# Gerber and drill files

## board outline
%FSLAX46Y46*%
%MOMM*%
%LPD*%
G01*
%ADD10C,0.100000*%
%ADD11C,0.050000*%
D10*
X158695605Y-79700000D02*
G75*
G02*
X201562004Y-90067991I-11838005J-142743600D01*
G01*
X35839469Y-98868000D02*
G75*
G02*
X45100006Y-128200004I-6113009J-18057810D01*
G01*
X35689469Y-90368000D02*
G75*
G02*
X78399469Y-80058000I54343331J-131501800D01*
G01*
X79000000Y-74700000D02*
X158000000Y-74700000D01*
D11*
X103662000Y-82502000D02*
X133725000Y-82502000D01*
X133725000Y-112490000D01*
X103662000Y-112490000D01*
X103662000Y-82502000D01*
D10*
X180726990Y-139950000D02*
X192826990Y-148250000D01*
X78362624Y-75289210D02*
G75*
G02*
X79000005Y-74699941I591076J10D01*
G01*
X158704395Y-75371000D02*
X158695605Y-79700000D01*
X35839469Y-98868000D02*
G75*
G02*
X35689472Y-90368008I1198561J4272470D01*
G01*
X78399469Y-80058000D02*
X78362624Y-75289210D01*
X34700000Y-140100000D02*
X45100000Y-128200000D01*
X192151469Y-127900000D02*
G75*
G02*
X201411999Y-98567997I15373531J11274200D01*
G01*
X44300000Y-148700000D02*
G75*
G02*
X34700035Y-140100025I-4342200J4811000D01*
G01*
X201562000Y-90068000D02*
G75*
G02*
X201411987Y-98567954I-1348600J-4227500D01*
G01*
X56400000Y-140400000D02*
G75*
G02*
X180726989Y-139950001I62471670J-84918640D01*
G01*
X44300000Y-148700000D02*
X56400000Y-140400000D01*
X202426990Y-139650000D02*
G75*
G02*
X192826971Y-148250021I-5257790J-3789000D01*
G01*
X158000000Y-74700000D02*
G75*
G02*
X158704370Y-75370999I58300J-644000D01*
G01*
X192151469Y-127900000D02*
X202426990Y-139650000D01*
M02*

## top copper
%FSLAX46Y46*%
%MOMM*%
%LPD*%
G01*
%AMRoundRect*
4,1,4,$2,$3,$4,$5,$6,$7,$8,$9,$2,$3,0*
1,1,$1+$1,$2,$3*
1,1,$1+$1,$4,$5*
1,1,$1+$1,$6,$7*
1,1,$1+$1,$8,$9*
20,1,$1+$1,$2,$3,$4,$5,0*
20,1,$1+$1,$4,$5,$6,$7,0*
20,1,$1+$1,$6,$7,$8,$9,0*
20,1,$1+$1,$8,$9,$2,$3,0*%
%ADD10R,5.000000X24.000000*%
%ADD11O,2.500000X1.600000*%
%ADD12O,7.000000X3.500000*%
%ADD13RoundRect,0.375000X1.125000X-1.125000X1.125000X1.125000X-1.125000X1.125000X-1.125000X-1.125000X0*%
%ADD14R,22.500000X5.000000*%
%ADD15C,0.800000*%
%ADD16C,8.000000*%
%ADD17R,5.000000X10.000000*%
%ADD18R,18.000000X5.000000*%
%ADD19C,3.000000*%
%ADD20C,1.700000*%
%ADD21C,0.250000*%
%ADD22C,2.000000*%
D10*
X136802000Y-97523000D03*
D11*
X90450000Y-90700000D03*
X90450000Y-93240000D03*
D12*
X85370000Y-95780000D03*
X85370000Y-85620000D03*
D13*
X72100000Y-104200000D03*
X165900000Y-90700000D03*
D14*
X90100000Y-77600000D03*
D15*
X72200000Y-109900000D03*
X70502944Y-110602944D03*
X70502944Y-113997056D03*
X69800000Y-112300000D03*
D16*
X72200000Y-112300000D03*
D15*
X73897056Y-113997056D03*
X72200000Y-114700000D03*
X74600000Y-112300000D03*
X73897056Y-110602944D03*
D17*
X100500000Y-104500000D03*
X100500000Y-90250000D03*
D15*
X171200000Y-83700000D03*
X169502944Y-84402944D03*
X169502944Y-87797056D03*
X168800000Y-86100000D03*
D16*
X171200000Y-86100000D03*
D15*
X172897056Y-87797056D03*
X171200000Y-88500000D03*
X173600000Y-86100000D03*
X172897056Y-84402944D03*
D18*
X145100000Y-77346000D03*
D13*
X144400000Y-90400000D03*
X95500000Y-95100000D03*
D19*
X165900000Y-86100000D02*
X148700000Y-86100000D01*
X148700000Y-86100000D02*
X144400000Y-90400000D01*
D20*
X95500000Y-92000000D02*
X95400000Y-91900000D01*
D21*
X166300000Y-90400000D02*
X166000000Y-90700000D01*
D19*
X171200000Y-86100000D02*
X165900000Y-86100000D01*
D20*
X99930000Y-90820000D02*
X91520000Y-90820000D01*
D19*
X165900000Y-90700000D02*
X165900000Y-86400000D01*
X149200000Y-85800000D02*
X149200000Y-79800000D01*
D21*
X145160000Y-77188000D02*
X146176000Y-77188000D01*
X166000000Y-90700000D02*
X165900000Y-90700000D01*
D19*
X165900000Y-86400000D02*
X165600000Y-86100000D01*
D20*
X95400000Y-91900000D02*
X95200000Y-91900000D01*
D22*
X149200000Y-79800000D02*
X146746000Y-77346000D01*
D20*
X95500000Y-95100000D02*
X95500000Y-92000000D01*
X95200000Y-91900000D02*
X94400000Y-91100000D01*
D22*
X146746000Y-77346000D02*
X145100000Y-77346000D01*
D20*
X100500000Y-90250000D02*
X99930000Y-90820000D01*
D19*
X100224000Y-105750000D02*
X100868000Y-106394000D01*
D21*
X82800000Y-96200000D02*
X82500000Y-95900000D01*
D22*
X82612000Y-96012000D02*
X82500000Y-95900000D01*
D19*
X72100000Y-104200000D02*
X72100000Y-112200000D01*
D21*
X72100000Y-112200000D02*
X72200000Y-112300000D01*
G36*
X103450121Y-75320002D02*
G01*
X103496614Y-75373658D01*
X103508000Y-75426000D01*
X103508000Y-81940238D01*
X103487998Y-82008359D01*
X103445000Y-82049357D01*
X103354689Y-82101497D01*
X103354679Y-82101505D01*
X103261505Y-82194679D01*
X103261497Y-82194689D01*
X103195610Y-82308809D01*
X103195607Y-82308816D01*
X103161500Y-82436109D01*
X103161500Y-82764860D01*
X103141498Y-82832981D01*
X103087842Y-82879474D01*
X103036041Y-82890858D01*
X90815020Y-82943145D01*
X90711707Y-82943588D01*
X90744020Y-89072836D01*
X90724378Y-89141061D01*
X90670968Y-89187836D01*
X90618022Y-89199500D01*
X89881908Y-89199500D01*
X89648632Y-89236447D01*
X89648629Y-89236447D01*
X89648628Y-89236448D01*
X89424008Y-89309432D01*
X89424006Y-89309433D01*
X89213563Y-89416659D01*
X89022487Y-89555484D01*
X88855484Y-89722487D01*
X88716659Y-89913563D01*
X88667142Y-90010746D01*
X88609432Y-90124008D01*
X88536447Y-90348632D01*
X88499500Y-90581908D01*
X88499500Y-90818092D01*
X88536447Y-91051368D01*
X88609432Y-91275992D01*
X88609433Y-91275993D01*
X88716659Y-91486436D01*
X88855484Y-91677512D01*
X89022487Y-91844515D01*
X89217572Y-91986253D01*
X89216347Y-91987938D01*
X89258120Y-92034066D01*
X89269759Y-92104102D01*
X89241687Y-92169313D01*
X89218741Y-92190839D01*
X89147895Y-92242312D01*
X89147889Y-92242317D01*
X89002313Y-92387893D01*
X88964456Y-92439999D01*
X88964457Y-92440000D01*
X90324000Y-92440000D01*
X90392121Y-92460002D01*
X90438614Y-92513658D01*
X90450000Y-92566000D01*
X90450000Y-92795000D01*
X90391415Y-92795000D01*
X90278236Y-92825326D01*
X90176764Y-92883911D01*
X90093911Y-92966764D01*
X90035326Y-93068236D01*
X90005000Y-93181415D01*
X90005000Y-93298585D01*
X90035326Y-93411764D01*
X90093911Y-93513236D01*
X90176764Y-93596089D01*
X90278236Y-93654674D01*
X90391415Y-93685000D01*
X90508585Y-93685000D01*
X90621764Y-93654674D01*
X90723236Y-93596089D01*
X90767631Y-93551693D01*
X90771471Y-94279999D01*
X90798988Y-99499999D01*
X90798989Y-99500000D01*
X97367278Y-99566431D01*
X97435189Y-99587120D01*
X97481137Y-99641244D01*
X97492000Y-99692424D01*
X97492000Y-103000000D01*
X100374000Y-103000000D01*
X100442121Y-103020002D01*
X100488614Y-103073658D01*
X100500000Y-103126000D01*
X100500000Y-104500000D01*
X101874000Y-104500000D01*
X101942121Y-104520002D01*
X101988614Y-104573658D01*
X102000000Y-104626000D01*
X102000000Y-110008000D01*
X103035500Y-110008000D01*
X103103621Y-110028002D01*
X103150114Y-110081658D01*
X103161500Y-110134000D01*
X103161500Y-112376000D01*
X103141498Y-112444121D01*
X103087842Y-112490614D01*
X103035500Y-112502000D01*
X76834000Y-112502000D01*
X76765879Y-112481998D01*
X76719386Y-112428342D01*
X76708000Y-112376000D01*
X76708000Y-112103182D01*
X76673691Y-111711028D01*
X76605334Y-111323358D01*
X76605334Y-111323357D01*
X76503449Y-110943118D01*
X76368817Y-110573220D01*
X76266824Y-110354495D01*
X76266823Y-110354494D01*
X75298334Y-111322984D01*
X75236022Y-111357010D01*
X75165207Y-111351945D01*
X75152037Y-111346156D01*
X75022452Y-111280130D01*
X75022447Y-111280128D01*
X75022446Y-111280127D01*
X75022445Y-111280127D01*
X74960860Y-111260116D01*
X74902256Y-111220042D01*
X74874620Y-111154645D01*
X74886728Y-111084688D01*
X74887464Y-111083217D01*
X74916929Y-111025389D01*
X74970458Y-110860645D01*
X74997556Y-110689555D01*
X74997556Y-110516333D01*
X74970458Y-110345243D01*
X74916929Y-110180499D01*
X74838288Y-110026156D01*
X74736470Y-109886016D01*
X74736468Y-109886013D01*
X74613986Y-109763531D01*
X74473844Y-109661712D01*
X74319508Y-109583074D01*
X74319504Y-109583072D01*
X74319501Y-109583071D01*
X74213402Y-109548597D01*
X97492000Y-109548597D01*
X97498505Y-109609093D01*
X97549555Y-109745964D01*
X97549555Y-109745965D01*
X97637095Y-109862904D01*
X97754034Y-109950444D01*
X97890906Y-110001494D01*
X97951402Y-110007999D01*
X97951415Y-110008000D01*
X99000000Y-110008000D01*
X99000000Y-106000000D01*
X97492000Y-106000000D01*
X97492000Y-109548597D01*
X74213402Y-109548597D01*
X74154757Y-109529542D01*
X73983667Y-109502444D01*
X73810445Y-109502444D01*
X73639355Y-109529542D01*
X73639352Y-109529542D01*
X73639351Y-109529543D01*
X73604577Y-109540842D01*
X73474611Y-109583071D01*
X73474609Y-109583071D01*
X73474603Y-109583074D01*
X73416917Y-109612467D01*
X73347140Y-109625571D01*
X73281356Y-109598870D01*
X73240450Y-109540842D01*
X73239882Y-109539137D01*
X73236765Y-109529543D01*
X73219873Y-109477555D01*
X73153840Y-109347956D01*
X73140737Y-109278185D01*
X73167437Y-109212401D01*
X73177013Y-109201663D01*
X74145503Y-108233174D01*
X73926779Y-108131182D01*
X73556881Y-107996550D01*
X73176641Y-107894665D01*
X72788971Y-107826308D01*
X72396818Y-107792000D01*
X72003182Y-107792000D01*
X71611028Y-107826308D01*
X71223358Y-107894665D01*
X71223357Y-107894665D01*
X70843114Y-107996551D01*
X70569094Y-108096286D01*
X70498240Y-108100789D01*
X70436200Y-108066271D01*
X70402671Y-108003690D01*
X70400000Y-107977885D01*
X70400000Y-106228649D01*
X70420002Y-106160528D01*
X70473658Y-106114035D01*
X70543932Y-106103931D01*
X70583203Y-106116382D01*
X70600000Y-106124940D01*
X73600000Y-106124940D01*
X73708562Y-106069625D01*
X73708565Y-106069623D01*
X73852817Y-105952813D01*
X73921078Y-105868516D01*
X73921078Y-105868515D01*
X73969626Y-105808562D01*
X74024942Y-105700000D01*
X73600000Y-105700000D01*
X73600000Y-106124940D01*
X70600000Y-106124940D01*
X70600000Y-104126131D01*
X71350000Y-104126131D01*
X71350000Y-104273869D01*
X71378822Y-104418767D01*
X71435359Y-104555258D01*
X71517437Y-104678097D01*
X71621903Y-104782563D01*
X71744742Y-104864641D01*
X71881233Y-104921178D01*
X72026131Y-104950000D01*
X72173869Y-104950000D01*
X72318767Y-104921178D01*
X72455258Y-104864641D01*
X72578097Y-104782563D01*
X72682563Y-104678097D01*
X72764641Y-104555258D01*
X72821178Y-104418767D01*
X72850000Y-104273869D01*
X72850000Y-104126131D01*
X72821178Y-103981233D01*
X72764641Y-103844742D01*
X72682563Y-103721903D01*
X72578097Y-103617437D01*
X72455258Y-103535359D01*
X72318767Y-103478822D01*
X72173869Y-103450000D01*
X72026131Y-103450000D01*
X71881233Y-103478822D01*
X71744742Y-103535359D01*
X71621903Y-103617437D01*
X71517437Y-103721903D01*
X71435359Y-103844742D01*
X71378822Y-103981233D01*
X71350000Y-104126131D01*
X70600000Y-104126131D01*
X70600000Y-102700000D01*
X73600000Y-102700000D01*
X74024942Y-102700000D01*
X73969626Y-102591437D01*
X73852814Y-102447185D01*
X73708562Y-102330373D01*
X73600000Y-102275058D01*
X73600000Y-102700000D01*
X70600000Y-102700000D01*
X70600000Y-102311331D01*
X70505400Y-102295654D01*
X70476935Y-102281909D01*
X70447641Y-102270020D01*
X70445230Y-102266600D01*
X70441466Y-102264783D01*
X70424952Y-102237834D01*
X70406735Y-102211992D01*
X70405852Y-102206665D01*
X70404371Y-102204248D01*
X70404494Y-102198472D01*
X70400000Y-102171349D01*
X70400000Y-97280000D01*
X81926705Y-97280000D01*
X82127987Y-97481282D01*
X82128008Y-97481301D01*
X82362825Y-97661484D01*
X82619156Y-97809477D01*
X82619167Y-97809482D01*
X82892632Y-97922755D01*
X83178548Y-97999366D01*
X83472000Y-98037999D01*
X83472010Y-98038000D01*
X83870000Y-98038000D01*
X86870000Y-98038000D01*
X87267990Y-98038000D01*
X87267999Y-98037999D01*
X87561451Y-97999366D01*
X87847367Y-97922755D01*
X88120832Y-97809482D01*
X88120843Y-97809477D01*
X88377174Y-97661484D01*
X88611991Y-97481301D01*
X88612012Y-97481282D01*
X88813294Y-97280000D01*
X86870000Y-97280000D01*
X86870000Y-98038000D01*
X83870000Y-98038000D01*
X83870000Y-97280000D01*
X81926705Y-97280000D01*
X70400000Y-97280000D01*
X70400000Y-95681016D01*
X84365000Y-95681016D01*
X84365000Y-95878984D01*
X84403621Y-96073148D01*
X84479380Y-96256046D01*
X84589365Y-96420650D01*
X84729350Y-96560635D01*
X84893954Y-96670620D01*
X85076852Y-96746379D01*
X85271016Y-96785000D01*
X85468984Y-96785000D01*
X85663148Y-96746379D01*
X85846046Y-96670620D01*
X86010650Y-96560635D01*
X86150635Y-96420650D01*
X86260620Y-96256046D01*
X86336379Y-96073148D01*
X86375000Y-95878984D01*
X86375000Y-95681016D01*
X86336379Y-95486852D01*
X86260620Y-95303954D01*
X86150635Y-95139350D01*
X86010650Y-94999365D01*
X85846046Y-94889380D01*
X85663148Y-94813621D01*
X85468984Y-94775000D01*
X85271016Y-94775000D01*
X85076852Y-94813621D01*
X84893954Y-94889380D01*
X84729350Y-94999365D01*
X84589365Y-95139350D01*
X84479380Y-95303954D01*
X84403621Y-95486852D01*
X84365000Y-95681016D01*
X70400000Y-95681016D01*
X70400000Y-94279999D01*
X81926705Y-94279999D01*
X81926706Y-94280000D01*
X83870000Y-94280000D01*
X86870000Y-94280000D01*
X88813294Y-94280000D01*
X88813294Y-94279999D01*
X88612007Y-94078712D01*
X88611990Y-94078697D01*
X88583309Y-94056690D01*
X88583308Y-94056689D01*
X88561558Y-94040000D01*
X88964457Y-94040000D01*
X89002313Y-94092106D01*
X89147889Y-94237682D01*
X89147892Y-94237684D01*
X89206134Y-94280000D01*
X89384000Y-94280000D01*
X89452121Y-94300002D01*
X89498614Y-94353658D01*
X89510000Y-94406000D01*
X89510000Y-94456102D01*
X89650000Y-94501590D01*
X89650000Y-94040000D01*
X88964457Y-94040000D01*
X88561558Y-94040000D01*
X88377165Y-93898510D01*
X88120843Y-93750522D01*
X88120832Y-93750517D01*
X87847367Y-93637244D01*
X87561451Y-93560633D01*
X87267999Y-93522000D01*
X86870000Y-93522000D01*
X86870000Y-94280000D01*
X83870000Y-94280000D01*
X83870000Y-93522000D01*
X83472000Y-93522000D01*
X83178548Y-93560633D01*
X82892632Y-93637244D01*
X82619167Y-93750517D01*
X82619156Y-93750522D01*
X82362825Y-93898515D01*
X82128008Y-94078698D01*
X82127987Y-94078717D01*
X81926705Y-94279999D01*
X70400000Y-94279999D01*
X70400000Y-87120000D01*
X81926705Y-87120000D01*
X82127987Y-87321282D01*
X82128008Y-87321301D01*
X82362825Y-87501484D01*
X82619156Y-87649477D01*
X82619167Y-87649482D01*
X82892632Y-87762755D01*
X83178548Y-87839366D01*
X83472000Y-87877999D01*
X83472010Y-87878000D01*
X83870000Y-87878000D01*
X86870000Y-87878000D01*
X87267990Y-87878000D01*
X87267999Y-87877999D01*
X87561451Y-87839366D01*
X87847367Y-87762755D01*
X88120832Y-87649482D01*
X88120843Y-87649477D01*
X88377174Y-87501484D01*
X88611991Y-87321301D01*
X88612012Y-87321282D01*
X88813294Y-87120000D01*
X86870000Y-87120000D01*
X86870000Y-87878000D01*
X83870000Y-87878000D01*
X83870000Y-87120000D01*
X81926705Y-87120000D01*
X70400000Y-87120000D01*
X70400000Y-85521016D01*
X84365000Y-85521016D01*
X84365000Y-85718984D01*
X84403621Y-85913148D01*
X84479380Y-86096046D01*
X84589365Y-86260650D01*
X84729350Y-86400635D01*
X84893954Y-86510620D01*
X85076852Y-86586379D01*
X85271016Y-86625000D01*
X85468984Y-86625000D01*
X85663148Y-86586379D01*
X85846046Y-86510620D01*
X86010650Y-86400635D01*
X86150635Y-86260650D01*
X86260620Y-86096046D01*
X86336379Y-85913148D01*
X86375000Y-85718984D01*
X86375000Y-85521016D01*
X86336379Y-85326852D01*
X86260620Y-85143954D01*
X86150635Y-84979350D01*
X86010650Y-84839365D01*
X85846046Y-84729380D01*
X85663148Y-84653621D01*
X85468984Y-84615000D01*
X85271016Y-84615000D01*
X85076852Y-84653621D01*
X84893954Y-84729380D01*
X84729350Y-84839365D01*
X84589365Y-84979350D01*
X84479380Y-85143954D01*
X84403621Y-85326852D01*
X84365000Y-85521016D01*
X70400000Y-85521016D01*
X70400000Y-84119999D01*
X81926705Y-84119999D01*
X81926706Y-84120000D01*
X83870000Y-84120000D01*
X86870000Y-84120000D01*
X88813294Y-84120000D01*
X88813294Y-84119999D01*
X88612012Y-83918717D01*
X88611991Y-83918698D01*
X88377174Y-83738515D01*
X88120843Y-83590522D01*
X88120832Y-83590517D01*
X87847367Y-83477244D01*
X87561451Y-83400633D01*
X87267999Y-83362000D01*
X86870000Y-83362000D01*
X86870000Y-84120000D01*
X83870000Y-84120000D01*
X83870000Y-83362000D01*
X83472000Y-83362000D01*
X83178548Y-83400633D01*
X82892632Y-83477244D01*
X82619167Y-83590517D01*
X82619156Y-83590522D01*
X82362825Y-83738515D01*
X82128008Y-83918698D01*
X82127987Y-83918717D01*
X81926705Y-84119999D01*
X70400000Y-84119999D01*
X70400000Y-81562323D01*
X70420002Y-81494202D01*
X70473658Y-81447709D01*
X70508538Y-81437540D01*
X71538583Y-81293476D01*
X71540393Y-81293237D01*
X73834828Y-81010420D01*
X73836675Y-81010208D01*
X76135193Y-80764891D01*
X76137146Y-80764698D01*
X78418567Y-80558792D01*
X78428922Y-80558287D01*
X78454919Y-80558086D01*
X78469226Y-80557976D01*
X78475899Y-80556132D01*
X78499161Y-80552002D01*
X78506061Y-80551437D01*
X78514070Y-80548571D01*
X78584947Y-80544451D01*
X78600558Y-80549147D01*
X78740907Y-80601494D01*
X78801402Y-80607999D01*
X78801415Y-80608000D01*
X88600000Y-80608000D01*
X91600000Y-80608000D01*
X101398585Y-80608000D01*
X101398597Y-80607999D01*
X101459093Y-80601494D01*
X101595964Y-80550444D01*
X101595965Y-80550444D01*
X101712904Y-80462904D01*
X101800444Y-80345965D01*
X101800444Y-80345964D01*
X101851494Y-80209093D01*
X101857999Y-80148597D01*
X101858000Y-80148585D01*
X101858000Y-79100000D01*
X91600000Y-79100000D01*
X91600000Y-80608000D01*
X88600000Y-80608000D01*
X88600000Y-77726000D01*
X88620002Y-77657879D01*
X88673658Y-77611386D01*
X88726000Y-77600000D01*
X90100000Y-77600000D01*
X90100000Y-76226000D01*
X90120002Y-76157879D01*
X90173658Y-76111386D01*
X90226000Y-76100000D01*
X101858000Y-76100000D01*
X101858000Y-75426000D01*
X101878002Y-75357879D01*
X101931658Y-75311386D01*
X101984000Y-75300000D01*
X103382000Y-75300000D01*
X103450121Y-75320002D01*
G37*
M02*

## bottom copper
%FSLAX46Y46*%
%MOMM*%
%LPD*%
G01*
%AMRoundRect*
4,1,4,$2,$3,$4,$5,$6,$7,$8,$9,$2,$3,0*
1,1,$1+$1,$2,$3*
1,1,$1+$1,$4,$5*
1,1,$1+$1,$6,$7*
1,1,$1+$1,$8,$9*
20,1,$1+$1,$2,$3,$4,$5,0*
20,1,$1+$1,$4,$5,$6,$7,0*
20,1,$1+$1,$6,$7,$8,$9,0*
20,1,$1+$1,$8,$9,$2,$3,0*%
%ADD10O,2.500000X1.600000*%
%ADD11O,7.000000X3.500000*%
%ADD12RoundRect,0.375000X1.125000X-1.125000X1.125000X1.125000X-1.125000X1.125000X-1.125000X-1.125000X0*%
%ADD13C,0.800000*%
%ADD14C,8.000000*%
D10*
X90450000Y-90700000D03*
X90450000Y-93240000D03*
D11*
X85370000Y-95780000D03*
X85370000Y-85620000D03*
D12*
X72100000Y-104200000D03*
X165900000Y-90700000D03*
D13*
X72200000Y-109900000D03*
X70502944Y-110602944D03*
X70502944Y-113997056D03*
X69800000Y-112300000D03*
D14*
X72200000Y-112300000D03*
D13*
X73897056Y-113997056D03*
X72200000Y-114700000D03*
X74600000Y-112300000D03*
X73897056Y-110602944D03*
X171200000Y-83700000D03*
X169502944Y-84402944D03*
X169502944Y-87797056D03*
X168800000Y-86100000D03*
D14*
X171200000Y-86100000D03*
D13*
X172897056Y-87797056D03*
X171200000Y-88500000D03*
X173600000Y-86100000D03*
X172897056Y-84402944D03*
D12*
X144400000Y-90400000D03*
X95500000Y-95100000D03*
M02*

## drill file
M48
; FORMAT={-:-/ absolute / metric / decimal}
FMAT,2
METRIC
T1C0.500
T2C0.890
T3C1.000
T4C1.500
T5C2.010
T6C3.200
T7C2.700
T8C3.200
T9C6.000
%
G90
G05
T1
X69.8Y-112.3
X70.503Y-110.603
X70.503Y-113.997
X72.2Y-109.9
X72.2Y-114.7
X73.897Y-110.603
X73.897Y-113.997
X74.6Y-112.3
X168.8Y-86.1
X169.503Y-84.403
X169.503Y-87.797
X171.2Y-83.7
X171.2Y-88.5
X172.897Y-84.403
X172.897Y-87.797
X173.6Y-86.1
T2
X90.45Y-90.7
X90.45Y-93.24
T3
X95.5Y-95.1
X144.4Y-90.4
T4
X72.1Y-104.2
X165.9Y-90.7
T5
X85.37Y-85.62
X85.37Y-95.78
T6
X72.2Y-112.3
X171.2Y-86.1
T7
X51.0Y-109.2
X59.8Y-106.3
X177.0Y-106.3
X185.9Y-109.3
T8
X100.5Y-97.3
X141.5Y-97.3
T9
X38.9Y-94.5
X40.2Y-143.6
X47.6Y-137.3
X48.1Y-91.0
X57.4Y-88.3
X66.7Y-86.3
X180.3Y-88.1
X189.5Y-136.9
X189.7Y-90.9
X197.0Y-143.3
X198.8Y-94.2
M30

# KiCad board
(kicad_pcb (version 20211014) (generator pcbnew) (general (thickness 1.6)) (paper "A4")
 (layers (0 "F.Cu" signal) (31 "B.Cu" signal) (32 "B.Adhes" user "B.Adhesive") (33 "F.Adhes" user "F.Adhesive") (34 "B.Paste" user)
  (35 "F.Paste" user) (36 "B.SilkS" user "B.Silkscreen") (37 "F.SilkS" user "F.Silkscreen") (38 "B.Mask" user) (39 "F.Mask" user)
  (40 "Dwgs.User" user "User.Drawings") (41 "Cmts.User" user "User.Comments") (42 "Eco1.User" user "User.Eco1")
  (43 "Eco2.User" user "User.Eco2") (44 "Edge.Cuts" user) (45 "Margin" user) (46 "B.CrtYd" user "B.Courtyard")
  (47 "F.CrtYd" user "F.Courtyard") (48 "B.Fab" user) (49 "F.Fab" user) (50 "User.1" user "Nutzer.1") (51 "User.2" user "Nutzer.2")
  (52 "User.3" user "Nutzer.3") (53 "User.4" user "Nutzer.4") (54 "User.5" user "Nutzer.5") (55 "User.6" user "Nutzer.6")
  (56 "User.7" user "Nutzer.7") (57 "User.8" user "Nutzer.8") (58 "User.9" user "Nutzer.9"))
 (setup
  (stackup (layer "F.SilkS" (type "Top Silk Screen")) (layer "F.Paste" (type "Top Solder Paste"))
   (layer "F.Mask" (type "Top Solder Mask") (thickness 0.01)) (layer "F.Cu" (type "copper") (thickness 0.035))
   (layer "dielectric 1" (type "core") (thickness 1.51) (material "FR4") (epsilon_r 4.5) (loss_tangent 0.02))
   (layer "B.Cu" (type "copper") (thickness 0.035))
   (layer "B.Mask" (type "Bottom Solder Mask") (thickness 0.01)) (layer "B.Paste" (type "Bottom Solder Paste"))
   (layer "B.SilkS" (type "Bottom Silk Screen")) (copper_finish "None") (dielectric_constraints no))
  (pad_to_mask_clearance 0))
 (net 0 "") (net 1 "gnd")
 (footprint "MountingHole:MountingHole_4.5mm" (layer "F.Cu") (at 57.4 88.3)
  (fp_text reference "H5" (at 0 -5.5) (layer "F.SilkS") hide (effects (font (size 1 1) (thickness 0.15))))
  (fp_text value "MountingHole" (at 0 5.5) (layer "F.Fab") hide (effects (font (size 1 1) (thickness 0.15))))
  (pad "" np_thru_hole circle (at 0 0) (size 6 6) (drill 6) (layers F&B.Cu *.Mask)))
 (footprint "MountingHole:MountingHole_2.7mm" (layer "F.Cu") (at 185.9 109.3)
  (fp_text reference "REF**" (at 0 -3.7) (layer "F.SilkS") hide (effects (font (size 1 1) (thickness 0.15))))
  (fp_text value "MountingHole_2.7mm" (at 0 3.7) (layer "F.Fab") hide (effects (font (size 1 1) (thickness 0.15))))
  (pad "" np_thru_hole circle (at 0 0) (size 2.7 2.7) (drill 2.7) (layers *.Cu *.Mask)))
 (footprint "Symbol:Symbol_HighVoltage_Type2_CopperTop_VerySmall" (layer "F.Cu") (at 174.9 94.2)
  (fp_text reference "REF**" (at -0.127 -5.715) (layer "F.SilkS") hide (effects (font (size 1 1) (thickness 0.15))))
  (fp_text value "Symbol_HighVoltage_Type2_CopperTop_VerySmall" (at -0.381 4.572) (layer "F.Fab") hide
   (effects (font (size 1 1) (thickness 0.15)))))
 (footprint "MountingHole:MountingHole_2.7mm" (layer "F.Cu") (at 59.8 106.3)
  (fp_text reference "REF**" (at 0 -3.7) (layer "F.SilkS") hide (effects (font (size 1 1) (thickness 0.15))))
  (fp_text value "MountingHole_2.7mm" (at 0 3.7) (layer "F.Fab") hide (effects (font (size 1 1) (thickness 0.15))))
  (pad "" np_thru_hole circle (at 0 0) (size 2.7 2.7) (drill 2.7) (layers *.Cu *.Mask)))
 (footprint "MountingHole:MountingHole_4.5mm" (layer "F.Cu") (at 38.9 94.5)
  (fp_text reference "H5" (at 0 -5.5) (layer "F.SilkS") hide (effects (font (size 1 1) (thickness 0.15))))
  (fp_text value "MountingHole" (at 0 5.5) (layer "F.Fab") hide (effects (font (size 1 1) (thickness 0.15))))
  (pad "" np_thru_hole circle (at 0 0) (size 6 6) (drill 6) (layers F&B.Cu *.Mask)))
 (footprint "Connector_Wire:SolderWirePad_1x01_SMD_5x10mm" (layer "F.Cu") (at 136.802 97.523 180)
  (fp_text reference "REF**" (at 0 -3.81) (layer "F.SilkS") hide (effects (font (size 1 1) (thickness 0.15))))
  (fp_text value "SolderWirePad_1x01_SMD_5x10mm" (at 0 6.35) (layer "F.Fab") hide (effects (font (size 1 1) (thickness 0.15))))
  (pad "1" smd rect (at 0 0 180) (size 5 24) (layers "F.Cu" "F.Mask")))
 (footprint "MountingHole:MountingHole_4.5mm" (layer "F.Cu") (at 180.3 88.1)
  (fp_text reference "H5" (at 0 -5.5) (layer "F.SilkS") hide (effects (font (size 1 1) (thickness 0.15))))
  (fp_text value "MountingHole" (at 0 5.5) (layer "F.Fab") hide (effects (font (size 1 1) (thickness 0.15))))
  (pad "" np_thru_hole circle (at 0 0) (size 6 6) (drill 6) (layers F&B.Cu *.Mask)))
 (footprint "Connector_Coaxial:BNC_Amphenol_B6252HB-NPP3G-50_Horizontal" (layer "F.Cu") (at 90.45 90.7 90)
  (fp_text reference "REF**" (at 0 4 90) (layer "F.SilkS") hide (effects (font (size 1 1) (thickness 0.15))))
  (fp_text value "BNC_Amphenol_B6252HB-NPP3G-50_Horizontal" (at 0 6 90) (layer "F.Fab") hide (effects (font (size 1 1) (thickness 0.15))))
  (pad "1" thru_hole oval (at 0 0 90) (size 1.6 2.5) (drill 0.89) (layers *.Cu *.Mask))
  (pad "2" thru_hole oval (at -2.54 0 90) (size 1.6 2.5) (drill 0.89) (layers *.Cu *.Mask) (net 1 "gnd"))
  (pad "2" thru_hole oval (at -5.08 -5.08 90) (size 3.5 7) (drill 2.01) (layers *.Cu *.Mask) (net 1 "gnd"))
  (pad "2" thru_hole oval (at 5.08 -5.08 90) (size 3.5 7) (drill 2.01) (layers *.Cu *.Mask) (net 1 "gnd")))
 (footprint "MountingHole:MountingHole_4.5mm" (layer "F.Cu") (at 189.7 90.9)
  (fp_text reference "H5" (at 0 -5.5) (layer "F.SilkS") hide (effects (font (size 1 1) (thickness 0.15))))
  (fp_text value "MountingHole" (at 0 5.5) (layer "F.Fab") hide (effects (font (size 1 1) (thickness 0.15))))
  (pad "" np_thru_hole circle (at 0 0) (size 6 6) (drill 6) (layers F&B.Cu *.Mask)))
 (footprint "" (layer "F.Cu") (at 72.1 104.2)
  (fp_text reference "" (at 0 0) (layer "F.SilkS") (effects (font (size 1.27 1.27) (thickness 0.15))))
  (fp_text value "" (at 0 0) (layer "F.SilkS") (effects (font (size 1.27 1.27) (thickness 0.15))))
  (pad "1" thru_hole roundrect (at 0 0 90) (size 3 3) (drill 1.5) (layers *.Cu *.Mask) (roundrect_rratio 0.125) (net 1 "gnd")))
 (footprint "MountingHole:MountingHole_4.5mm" (layer "F.Cu") (at 40.2 143.6)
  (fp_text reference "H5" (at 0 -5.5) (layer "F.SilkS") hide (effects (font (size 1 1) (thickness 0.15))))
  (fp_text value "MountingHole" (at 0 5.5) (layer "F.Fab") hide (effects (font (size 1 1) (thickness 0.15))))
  (pad "" np_thru_hole circle (at 0 0) (size 6 6) (drill 6) (layers F&B.Cu *.Mask)))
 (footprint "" (layer "F.Cu") (at 165.9 90.7)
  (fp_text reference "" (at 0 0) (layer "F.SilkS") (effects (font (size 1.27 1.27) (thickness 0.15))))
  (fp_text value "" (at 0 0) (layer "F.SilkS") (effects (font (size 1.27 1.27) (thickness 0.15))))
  (pad "1" thru_hole roundrect (at 0 0 90) (size 3 3) (drill 1.5) (layers *.Cu *.Mask) (roundrect_rratio 0.125)))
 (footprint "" (layer "F.Cu") (at 90.1 77.6)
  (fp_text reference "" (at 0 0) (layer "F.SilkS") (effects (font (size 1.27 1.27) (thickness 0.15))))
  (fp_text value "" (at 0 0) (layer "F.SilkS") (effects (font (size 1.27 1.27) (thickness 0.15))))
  (pad "1" smd rect (at 0 0 180) (size 22.5 5) (layers "F.Cu" "F.Mask") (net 1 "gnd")))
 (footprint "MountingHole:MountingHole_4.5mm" (layer "F.Cu") (at 197 143.3)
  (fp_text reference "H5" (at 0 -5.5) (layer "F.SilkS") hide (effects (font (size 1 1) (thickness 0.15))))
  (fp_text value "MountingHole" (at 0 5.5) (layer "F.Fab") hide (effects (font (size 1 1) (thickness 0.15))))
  (pad "" np_thru_hole circle (at 0 0) (size 6 6) (drill 6) (layers F&B.Cu *.Mask)))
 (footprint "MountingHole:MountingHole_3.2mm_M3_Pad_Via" (layer "F.Cu") (at 72.2 112.3)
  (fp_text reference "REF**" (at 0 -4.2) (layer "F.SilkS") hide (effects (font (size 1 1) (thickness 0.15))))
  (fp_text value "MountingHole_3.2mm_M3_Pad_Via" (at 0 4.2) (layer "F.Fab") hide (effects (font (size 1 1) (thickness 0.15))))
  (pad "1" thru_hole circle (at 0 -2.4) (size 0.8 0.8) (drill 0.5) (layers *.Cu *.Mask))
  (pad "1" thru_hole circle (at -1.697056 -1.697056) (size 0.8 0.8) (drill 0.5) (layers *.Cu *.Mask))
  (pad "1" thru_hole circle (at -1.697056 1.697056) (size 0.8 0.8) (drill 0.5) (layers *.Cu *.Mask))
  (pad "1" thru_hole circle (at -2.4 0) (size 0.8 0.8) (drill 0.5) (layers *.Cu *.Mask))
  (pad "1" thru_hole circle (at 0 0) (size 8 8) (drill 3.2) (layers *.Cu *.Mask) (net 1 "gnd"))
  (pad "1" thru_hole circle (at 1.697056 1.697056) (size 0.8 0.8) (drill 0.5) (layers *.Cu *.Mask))
  (pad "1" thru_hole circle (at 0 2.4) (size 0.8 0.8) (drill 0.5) (layers *.Cu *.Mask))
  (pad "1" thru_hole circle (at 2.4 0) (size 0.8 0.8) (drill 0.5) (layers *.Cu *.Mask))
  (pad "1" thru_hole circle (at 1.697056 -1.697056) (size 0.8 0.8) (drill 0.5) (layers *.Cu *.Mask)))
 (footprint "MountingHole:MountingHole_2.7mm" (layer "F.Cu") (at 177 106.3)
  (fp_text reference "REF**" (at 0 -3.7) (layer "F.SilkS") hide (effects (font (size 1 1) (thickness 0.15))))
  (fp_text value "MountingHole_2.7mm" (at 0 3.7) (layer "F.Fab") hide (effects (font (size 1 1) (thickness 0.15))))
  (pad "" np_thru_hole circle (at 0 0) (size 2.7 2.7) (drill 2.7) (layers *.Cu *.Mask)))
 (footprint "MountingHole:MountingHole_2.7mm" (layer "F.Cu") (at 51 109.2)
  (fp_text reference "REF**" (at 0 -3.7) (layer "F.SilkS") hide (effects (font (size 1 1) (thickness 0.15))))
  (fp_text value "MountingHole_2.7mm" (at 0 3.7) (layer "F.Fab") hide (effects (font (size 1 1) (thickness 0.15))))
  (pad "" np_thru_hole circle (at 0 0) (size 2.7 2.7) (drill 2.7) (layers *.Cu *.Mask)))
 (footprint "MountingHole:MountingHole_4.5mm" (layer "F.Cu") (at 198.8 94.2)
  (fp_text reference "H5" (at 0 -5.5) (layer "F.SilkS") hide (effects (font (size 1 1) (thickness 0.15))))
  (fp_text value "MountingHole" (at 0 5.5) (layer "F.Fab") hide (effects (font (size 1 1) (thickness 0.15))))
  (pad "" np_thru_hole circle (at 0 0) (size 6 6) (drill 6) (layers F&B.Cu *.Mask)))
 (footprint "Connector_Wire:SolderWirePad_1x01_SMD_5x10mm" (layer "F.Cu") (at 100.5 104.5 180)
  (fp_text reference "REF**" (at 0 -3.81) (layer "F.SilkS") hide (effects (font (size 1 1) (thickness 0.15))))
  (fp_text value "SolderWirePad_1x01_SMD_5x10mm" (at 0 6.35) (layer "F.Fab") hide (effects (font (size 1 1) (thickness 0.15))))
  (pad "1" smd rect (at 0 0 180) (size 5 10) (layers "F.Cu" "F.Mask") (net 1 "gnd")))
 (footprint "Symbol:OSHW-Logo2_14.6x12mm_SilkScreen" (layer "F.Cu") (at 59.7 120.2)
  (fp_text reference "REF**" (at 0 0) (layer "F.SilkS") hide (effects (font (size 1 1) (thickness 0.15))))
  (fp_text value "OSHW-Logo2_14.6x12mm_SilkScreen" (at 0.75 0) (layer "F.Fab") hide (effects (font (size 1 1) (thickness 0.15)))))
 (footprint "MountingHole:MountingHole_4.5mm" (layer "F.Cu") (at 66.7 86.3)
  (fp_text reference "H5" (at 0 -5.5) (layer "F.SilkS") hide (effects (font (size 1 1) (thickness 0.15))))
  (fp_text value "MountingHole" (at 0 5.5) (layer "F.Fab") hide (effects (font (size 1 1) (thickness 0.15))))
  (pad "" np_thru_hole circle (at 0 0) (size 6 6) (drill 6) (layers F&B.Cu *.Mask)))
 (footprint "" (layer "F.Cu") (at 100.5 90.25 90)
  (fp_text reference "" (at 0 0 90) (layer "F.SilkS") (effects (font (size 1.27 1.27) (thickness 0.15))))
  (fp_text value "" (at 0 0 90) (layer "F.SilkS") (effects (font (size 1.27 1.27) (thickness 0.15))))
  (pad "1" smd rect (at 0 0 180) (size 5 10) (layers "F.Cu" "F.Mask")))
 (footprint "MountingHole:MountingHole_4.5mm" (layer "F.Cu") (at 189.5 136.9)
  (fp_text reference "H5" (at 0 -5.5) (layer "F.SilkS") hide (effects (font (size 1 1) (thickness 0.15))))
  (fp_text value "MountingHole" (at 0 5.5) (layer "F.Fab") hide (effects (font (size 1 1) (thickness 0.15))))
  (pad "" np_thru_hole circle (at 0 0) (size 6 6) (drill 6) (layers F&B.Cu *.Mask)))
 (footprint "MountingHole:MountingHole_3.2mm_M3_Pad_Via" (layer "F.Cu") (at 171.2 86.1)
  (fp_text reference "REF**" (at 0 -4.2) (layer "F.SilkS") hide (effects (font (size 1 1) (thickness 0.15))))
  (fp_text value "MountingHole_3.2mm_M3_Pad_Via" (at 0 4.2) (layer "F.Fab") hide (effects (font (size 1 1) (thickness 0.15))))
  (pad "1" thru_hole circle (at 0 -2.4) (size 0.8 0.8) (drill 0.5) (layers *.Cu *.Mask))
  (pad "1" thru_hole circle (at -1.697056 -1.697056) (size 0.8 0.8) (drill 0.5) (layers *.Cu *.Mask))
  (pad "1" thru_hole circle (at -1.697056 1.697056) (size 0.8 0.8) (drill 0.5) (layers *.Cu *.Mask))
  (pad "1" thru_hole circle (at -2.4 0) (size 0.8 0.8) (drill 0.5) (layers *.Cu *.Mask))
  (pad "1" thru_hole circle (at 0 0) (size 8 8) (drill 3.2) (layers *.Cu *.Mask))
  (pad "1" thru_hole circle (at 1.697056 1.697056) (size 0.8 0.8) (drill 0.5) (layers *.Cu *.Mask))
  (pad "1" thru_hole circle (at 0 2.4) (size 0.8 0.8) (drill 0.5) (layers *.Cu *.Mask))
  (pad "1" thru_hole circle (at 2.4 0) (size 0.8 0.8) (drill 0.5) (layers *.Cu *.Mask))
  (pad "1" thru_hole circle (at 1.697056 -1.697056) (size 0.8 0.8) (drill 0.5) (layers *.Cu *.Mask)))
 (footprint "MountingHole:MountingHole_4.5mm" (layer "F.Cu") (at 48.1 91)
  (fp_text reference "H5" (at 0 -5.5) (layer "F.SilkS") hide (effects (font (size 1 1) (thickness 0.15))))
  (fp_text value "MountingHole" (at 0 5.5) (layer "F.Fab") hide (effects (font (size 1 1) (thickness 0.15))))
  (pad "" np_thru_hole circle (at 0 0) (size 6 6) (drill 6) (layers F&B.Cu *.Mask)))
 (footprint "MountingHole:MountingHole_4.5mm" (layer "F.Cu") (at 47.6 137.3)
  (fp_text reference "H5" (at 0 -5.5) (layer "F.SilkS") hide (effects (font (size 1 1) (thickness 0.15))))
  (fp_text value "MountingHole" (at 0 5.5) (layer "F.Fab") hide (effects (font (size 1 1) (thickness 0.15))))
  (pad "" np_thru_hole circle (at 0 0) (size 6 6) (drill 6) (layers F&B.Cu *.Mask)))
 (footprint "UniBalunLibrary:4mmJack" (layer "B.Cu") (at 145.354 77.6)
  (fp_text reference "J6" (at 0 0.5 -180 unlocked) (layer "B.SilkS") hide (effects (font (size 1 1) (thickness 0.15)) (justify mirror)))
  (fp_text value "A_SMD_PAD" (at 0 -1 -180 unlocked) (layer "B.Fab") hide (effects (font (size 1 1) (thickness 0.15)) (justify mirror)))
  (pad "1" smd rect (at -0.254 -0.254) (size 18 5) (layers "F.Cu" "F.Mask")))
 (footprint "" (layer "B.Cu") (at 141.5 97.3 90)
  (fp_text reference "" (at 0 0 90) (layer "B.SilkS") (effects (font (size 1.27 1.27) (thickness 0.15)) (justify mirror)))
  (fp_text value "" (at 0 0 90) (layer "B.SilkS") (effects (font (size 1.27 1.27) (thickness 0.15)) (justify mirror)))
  (pad "" np_thru_hole circle (at 0 0 90) (size 3.2 3.2) (drill 3.2) (layers *.Cu *.Mask)))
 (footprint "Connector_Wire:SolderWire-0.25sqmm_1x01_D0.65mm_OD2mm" (layer "B.Cu") (at 144.4 90.4 90)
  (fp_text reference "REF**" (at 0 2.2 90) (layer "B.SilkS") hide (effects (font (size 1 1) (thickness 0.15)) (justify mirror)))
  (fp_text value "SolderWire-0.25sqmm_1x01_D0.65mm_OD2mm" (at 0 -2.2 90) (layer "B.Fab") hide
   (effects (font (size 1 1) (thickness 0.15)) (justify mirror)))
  (pad "1" thru_hole roundrect (at 0 0 90) (size 3 3) (drill 1) (layers *.Cu *.Mask) (roundrect_rratio 0.125)))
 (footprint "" (layer "B.Cu") (at 95.5 95.1 90)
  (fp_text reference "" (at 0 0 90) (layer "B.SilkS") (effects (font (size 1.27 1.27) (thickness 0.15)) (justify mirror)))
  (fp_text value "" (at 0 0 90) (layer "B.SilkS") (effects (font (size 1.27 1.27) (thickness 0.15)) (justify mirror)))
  (pad "1" thru_hole roundrect (at 0 0 90) (size 3 3) (drill 1) (layers *.Cu *.Mask) (roundrect_rratio 0.125)))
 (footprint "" (layer "B.Cu") (at 100.5 97.3 90)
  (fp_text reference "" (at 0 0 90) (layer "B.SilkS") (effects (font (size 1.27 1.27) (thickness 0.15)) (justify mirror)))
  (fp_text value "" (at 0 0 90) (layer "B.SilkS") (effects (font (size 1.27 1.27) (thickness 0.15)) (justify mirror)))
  (pad "" np_thru_hole circle (at 0 0 90) (size 3.2 3.2) (drill 3.2) (layers *.Cu *.Mask)))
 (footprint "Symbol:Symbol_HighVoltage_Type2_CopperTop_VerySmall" (layer "B.Cu") (at 175.1 94.2 180)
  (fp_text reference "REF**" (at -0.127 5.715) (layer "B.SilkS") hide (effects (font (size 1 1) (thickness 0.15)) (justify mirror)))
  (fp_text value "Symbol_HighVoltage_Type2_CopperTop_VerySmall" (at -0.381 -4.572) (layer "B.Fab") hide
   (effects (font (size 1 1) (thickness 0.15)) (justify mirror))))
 (gr_arc (start 158.695605 79.7) (mid 180.530241 83.224257) (end 201.562 90.068) (layer "Edge.Cuts") (width 0.1))
 (gr_arc (start 35.839469 98.868) (mid 47.90638 111.186145) (end 45.1 128.2) (layer "Edge.Cuts") (width 0.1))
 (gr_arc (start 35.689469 90.368) (mid 56.644119 83.554519) (end 78.399469 80.058) (layer "Edge.Cuts") (width 0.1))
 (gr_line (start 79 74.7) (end 158 74.7) (layer "Edge.Cuts") (width 0.1))
 (gr_rect (start 133.725 82.502) (end 103.662 112.49) (layer "Edge.Cuts") (width 0.05) (fill none))
 (gr_line (start 180.72699 139.95) (end 192.82699 148.25) (layer "Edge.Cuts") (width 0.1))
 (gr_arc (start 78.362624 75.28921) (mid 78.552454 74.855213) (end 79 74.7) (layer "Edge.Cuts") (width 0.1))
 (gr_line (start 158.704395 75.371) (end 158.695605 79.7) (layer "Edge.Cuts") (width 0.1))
 (gr_arc (start 35.839469 98.868) (mid 32.601313 94.67382) (end 35.689469 90.368) (layer "Edge.Cuts") (width 0.1))
 (gr_line (start 78.399469 80.058) (end 78.362624 75.28921) (layer "Edge.Cuts") (width 0.1))
 (gr_line (start 34.7 140.1) (end 45.1 128.2) (layer "Edge.Cuts") (width 0.1))
 (gr_arc (start 192.151469 127.9) (mid 189.345089 110.886145) (end 201.412 98.568) (layer "Edge.Cuts") (width 0.1))
 (gr_arc (start 44.3 148.7) (mid 35.633485 148.716109) (end 34.7 140.1) (layer "Edge.Cuts") (width 0.1))
 (gr_arc (start 201.562 90.068) (mid 204.650156 94.37382) (end 201.412 98.568) (layer "Edge.Cuts") (width 0.1))
 (gr_arc (start 56.4 140.4) (mid 118.490099 119.896917) (end 180.72699 139.95) (layer "Edge.Cuts") (width 0.1))
 (gr_line (start 44.3 148.7) (end 56.4 140.4) (layer "Edge.Cuts") (width 0.1))
 (gr_arc (start 202.42699 139.65) (mid 201.493505 148.266109) (end 192.82699 148.25) (layer "Edge.Cuts") (width 0.1))
 (gr_arc (start 158 74.7) (mid 158.504319 74.875807) (end 158.704395 75.371) (layer "Edge.Cuts") (width 0.1))
 (gr_line (start 192.151469 127.9) (end 202.42699 139.65) (layer "Edge.Cuts") (width 0.1))
 (segment (start 165.9 86.1) (end 148.7 86.1) (width 3) (layer "F.Cu") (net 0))
 (segment (start 148.7 86.1) (end 144.4 90.4) (width 3) (layer "F.Cu") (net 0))
 (segment (start 95.5 92) (end 95.4 91.9) (width 1.7) (layer "F.Cu") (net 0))
 (segment (start 166.3 90.4) (end 166 90.7) (width 0.25) (layer "F.Cu") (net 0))
 (segment (start 171.2 86.1) (end 165.9 86.1) (width 3) (layer "F.Cu") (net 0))
 (segment (start 99.93 90.82) (end 91.52 90.82) (width 1.7) (layer "F.Cu") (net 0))
 (segment (start 165.9 90.7) (end 165.9 86.4) (width 3) (layer "F.Cu") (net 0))
 (segment (start 149.2 85.8) (end 149.2 79.8) (width 3) (layer "F.Cu") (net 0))
 (segment (start 145.16 77.188) (end 146.176 77.188) (width 0.25) (layer "F.Cu") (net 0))
 (segment (start 166 90.7) (end 165.9 90.7) (width 0.25) (layer "F.Cu") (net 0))
 (segment (start 165.9 86.4) (end 165.6 86.1) (width 3) (layer "F.Cu") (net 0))
 (segment (start 95.4 91.9) (end 95.2 91.9) (width 1.7) (layer "F.Cu") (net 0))
 (segment (start 149.2 79.8) (end 146.746 77.346) (width 2) (layer "F.Cu") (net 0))
 (segment (start 95.5 95.1) (end 95.5 92) (width 1.7) (layer "F.Cu") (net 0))
 (segment (start 95.2 91.9) (end 94.4 91.1) (width 1.7) (layer "F.Cu") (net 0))
 (segment (start 146.746 77.346) (end 145.1 77.346) (width 2) (layer "F.Cu") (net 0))
 (segment (start 100.5 90.25) (end 99.93 90.82) (width 1.7) (layer "F.Cu") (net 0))
 (segment (start 100.224 105.75) (end 100.868 106.394) (width 3) (layer "F.Cu") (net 1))
 (segment (start 82.8 96.2) (end 82.5 95.9) (width 0.25) (layer "F.Cu") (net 1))
 (segment (start 82.612 96.012) (end 82.5 95.9) (width 2) (layer "F.Cu") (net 1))
 (segment (start 72.1 104.2) (end 72.1 112.2) (width 3) (layer "F.Cu") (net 1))
 (segment (start 72.1 112.2) (end 72.2 112.3) (width 0.25) (layer "F.Cu") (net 1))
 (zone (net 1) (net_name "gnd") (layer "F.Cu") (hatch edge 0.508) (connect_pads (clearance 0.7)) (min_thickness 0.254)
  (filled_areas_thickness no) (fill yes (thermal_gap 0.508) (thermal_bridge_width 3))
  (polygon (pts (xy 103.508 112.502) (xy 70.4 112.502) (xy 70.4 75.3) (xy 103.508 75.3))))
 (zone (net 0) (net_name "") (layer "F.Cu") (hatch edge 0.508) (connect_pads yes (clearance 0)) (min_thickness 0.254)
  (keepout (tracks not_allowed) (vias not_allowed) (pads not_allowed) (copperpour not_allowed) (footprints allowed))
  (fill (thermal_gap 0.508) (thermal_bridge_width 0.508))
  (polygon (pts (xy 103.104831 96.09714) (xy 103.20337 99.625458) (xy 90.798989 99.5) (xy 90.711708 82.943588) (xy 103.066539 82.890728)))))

